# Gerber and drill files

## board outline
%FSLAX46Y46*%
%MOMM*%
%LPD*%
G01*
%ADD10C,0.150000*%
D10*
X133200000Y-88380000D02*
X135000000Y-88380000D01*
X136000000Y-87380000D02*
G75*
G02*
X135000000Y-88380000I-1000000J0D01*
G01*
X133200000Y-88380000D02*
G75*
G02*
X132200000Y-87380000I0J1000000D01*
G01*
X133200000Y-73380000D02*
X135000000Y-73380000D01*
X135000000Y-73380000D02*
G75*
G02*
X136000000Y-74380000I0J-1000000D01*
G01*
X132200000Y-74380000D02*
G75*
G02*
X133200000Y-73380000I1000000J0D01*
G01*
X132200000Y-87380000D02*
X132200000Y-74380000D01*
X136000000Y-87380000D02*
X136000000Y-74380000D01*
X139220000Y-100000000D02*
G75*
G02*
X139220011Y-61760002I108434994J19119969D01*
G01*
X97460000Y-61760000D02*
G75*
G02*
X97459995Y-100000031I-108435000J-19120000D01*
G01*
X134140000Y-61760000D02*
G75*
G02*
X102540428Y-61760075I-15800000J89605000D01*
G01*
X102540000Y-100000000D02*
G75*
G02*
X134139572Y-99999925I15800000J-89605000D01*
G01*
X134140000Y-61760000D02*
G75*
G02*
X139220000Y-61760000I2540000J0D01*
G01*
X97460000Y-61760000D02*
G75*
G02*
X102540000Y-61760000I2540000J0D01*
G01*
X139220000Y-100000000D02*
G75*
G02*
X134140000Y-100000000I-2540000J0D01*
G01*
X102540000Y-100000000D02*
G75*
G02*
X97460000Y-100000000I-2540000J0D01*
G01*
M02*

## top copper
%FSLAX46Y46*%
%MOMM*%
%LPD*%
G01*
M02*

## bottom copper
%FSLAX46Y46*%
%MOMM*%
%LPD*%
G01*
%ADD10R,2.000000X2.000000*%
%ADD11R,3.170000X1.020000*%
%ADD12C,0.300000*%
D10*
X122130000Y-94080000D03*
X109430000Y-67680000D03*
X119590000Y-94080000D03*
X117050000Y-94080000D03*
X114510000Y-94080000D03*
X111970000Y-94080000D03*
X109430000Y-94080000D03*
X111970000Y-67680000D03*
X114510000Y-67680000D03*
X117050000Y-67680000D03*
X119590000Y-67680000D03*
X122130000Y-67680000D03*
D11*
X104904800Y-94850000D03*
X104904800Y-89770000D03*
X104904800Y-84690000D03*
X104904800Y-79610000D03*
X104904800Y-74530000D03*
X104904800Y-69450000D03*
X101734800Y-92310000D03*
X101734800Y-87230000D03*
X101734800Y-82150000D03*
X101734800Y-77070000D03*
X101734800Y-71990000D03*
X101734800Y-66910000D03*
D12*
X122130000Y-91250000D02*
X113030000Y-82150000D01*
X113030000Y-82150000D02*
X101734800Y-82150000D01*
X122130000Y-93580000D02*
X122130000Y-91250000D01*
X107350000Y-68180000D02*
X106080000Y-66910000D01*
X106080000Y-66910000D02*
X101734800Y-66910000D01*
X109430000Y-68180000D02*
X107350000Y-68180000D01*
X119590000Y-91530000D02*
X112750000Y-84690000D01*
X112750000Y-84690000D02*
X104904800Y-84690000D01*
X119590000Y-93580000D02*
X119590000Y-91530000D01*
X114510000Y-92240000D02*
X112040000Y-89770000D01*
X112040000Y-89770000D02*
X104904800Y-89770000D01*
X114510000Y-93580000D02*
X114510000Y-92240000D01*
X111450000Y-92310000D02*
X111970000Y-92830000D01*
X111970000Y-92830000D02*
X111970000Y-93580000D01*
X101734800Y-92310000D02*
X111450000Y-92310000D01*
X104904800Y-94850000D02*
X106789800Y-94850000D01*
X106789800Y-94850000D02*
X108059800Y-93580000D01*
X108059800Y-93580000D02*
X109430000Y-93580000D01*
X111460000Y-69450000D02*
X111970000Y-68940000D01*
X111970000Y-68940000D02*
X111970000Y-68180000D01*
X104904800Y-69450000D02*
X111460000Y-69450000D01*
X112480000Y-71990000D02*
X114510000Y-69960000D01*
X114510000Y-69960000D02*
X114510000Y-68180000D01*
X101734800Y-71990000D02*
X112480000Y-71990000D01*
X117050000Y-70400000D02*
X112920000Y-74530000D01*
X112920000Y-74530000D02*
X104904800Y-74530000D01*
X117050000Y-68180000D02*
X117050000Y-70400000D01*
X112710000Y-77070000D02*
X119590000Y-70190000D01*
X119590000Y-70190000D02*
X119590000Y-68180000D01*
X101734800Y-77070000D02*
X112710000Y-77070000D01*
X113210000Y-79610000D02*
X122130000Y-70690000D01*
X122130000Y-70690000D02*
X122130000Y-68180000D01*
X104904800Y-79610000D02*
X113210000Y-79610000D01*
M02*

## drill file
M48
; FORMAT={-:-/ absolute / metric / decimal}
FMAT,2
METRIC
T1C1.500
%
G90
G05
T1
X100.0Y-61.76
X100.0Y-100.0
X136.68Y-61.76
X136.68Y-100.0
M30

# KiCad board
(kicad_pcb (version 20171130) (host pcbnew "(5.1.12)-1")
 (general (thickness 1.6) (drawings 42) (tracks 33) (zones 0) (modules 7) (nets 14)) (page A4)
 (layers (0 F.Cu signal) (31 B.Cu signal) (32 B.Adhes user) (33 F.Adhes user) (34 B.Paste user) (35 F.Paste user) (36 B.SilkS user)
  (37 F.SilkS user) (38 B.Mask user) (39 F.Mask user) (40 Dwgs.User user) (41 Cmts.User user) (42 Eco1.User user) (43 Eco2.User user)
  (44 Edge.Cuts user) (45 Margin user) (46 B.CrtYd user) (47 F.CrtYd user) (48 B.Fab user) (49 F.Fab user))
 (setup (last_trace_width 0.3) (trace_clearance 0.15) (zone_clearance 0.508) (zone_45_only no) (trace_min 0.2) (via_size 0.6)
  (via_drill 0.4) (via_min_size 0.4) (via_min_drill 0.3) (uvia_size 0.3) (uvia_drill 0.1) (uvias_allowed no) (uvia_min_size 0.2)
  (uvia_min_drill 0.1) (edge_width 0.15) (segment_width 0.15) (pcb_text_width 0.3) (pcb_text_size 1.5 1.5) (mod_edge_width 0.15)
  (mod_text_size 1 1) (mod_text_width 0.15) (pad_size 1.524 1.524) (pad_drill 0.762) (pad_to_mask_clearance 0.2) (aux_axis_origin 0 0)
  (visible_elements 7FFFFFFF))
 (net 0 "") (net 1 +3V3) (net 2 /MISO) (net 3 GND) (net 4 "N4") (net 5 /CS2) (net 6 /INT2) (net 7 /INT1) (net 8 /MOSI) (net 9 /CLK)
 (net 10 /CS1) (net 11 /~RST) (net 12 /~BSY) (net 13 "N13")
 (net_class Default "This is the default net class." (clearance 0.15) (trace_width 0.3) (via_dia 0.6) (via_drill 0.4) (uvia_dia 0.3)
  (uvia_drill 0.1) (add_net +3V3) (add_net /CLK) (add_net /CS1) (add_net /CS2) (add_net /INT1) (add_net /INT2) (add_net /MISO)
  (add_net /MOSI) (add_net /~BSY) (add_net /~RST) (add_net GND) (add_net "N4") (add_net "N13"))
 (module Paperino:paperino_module (layer B.Cu) (at 118.73 80.88 90)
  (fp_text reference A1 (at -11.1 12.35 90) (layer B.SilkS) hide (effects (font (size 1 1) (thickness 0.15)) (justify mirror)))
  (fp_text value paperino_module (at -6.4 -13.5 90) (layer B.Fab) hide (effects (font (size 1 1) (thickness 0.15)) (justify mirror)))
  (pad 1 smd rect (at -12.7 3.4 90) (size 2 2) (drill (offset -0.5 0)) (layers B.Cu B.Paste B.Mask) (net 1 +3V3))
  (pad 7 smd rect (at 12.7 -9.3 90) (size 2 2) (drill (offset 0.5 0)) (layers B.Cu B.Paste B.Mask) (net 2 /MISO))
  (pad 2 smd rect (at -12.7 0.86 90) (size 2 2) (drill (offset -0.5 0)) (layers B.Cu B.Paste B.Mask) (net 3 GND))
  (pad 3 smd rect (at -12.7 -1.68 90) (size 2 2) (drill (offset -0.5 0)) (layers B.Cu B.Paste B.Mask) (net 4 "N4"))
  (pad 4 smd rect (at -12.7 -4.22 90) (size 2 2) (drill (offset -0.5 0)) (layers B.Cu B.Paste B.Mask) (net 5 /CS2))
  (pad 5 smd rect (at -12.7 -6.76 90) (size 2 2) (drill (offset -0.5 0)) (layers B.Cu B.Paste B.Mask) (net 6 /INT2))
  (pad 6 smd rect (at -12.7 -9.3 90) (size 2 2) (drill (offset -0.5 0)) (layers B.Cu B.Paste B.Mask) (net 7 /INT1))
  (pad 8 smd rect (at 12.7 -6.76 90) (size 2 2) (drill (offset 0.5 0)) (layers B.Cu B.Paste B.Mask) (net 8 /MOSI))
  (pad 9 smd rect (at 12.7 -4.22 90) (size 2 2) (drill (offset 0.5 0)) (layers B.Cu B.Paste B.Mask) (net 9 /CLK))
  (pad 10 smd rect (at 12.7 -1.68 90) (size 2 2) (drill (offset 0.5 0)) (layers B.Cu B.Paste B.Mask) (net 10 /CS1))
  (pad 11 smd rect (at 12.7 0.86 90) (size 2 2) (drill (offset 0.5 0)) (layers B.Cu B.Paste B.Mask) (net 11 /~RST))
  (pad 12 smd rect (at 12.7 3.4 90) (size 2 2) (drill (offset 0.5 0)) (layers B.Cu B.Paste B.Mask) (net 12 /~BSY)))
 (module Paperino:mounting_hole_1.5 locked (layer F.Cu) (at 100 100)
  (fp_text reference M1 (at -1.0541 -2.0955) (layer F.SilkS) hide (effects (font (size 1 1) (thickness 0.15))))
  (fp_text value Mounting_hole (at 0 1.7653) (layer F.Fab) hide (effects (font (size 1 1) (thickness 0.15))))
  (pad "" np_thru_hole circle (at 0 0) (size 1.5 1.5) (drill 1.5) (layers *.Cu *.Mask)))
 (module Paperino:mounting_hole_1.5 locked (layer F.Cu) (at 136.68 100)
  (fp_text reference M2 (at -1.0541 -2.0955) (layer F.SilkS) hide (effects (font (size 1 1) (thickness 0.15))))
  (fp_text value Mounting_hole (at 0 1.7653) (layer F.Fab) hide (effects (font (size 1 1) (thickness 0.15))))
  (pad "" np_thru_hole circle (at 0 0) (size 1.5 1.5) (drill 1.5) (layers *.Cu *.Mask)))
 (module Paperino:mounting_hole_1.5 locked (layer F.Cu) (at 100 61.76)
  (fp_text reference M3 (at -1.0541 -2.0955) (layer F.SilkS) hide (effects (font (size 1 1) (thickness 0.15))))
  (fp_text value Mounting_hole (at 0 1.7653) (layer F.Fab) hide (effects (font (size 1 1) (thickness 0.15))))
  (pad "" np_thru_hole circle (at 0 0) (size 1.5 1.5) (drill 1.5) (layers *.Cu *.Mask)))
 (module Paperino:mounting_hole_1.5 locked (layer F.Cu) (at 136.68 61.76)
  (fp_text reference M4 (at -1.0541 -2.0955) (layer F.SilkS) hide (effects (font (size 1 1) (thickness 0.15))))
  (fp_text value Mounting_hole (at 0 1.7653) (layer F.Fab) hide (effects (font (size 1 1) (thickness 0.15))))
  (pad "" np_thru_hole circle (at 0 0) (size 1.5 1.5) (drill 1.5) (layers *.Cu *.Mask)))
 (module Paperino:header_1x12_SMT (layer B.Cu) (at 103.32 80.88 90)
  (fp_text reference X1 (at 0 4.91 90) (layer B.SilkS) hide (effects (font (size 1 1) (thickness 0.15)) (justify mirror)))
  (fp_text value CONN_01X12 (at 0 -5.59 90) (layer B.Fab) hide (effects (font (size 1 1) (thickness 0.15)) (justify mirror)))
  (pad 1 smd rect (at -13.97 1.5848 90) (size 1.02 3.17) (layers B.Cu B.Paste B.Mask) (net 7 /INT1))
  (pad 3 smd rect (at -8.89 1.5848 90) (size 1.02 3.17) (layers B.Cu B.Paste B.Mask) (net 5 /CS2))
  (pad 5 smd rect (at -3.81 1.5848 90) (size 1.02 3.17) (layers B.Cu B.Paste B.Mask) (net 3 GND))
  (pad 7 smd rect (at 1.27 1.5848 90) (size 1.02 3.17) (layers B.Cu B.Paste B.Mask) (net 12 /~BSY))
  (pad 9 smd rect (at 6.35 1.5848 90) (size 1.02 3.17) (layers B.Cu B.Paste B.Mask) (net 10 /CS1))
  (pad 11 smd rect (at 11.43 1.5848 90) (size 1.02 3.17) (layers B.Cu B.Paste B.Mask) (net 8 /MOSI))
  (pad 2 smd rect (at -11.43 -1.5852 90) (size 1.02 3.17) (layers B.Cu B.Paste B.Mask) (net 6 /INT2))
  (pad 4 smd rect (at -6.35 -1.5852 90) (size 1.02 3.17) (layers B.Cu B.Paste B.Mask) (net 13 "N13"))
  (pad 6 smd rect (at -1.27 -1.5852 90) (size 1.02 3.17) (layers B.Cu B.Paste B.Mask) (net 1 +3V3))
  (pad 8 smd rect (at 3.81 -1.5852 90) (size 1.02 3.17) (layers B.Cu B.Paste B.Mask) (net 11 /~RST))
  (pad 10 smd rect (at 8.89 -1.5852 90) (size 1.02 3.17) (layers B.Cu B.Paste B.Mask) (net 9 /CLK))
  (pad 12 smd rect (at 13.97 -1.5852 90) (size 1.02 3.17) (layers B.Cu B.Paste B.Mask) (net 2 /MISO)))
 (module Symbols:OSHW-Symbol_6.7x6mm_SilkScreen (layer F.Cu) (at 133.66 67.9 90)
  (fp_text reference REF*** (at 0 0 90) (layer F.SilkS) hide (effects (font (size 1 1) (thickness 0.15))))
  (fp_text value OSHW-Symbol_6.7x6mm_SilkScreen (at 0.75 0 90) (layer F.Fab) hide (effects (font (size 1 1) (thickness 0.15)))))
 (gr_line (start 133.2 88.38) (end 135 88.38) (layer Edge.Cuts) (width 0.15))
 (gr_arc (start 135 87.38) (end 136 87.38) (angle 90) (layer Edge.Cuts) (width 0.15))
 (gr_arc (start 133.2 87.38) (end 133.2 88.38) (angle 90) (layer Edge.Cuts) (width 0.15))
 (gr_line (start 133.2 73.38) (end 135 73.38) (layer Edge.Cuts) (width 0.15))
 (gr_arc (start 135 74.38) (end 135 73.38) (angle 90) (layer Edge.Cuts) (width 0.15))
 (gr_arc (start 133.2 74.38) (end 132.2 74.38) (angle 90) (layer Edge.Cuts) (width 0.15))
 (gr_line (start 132.2 87.38) (end 132.2 74.38) (layer Edge.Cuts) (width 0.15))
 (gr_line (start 136 87.38) (end 136 74.38) (layer Edge.Cuts) (width 0.15))
 (gr_arc (start 247.654994 80.880031) (end 139.22 100) (angle 19.9999845) (layer Edge.Cuts) (width 0.15))
 (gr_arc (start -10.975 80.88) (end 97.46 61.76) (angle 20) (layer Edge.Cuts) (width 0.15))
 (gr_arc (start 118.34 -27.845) (end 134.14 61.76) (angle 20) (layer Edge.Cuts) (width 0.15))
 (gr_arc (start 118.34 189.605) (end 102.54 100) (angle 20) (layer Edge.Cuts) (width 0.15))
 (gr_arc (start 136.68 61.76) (end 134.14 61.76) (angle 180) (layer Edge.Cuts) (width 0.15))
 (gr_arc (start 100 61.76) (end 97.46 61.76) (angle 180) (layer Edge.Cuts) (width 0.15))
 (gr_arc (start 136.68 100) (end 139.22 100) (angle 180) (layer Edge.Cuts) (width 0.15))
 (gr_arc (start 100 100) (end 102.54 100) (angle 180) (layer Edge.Cuts) (width 0.15))
 (segment (start 122.13 91.25) (end 113.03 82.15) (width 0.3) (layer B.Cu) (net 1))
 (segment (start 113.03 82.15) (end 101.7348 82.15) (width 0.3) (layer B.Cu) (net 1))
 (segment (start 122.13 93.58) (end 122.13 91.25) (width 0.3) (layer B.Cu) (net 1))
 (segment (start 107.35 68.18) (end 106.08 66.91) (width 0.3) (layer B.Cu) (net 2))
 (segment (start 106.08 66.91) (end 101.7348 66.91) (width 0.3) (layer B.Cu) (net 2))
 (segment (start 109.43 68.18) (end 107.35 68.18) (width 0.3) (layer B.Cu) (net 2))
 (segment (start 119.59 91.53) (end 112.75 84.69) (width 0.3) (layer B.Cu) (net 3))
 (segment (start 112.75 84.69) (end 104.9048 84.69) (width 0.3) (layer B.Cu) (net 3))
 (segment (start 119.59 93.58) (end 119.59 91.53) (width 0.3) (layer B.Cu) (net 3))
 (segment (start 114.51 92.24) (end 112.04 89.77) (width 0.3) (layer B.Cu) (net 5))
 (segment (start 112.04 89.77) (end 104.9048 89.77) (width 0.3) (layer B.Cu) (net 5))
 (segment (start 114.51 93.58) (end 114.51 92.24) (width 0.3) (layer B.Cu) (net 5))
 (segment (start 111.45 92.31) (end 111.97 92.83) (width 0.3) (layer B.Cu) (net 6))
 (segment (start 111.97 92.83) (end 111.97 93.58) (width 0.3) (layer B.Cu) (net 6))
 (segment (start 101.7348 92.31) (end 111.45 92.31) (width 0.3) (layer B.Cu) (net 6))
 (segment (start 104.9048 94.85) (end 106.7898 94.85) (width 0.3) (layer B.Cu) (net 7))
 (segment (start 106.7898 94.85) (end 108.0598 93.58) (width 0.3) (layer B.Cu) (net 7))
 (segment (start 108.0598 93.58) (end 109.43 93.58) (width 0.3) (layer B.Cu) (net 7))
 (segment (start 111.46 69.45) (end 111.97 68.94) (width 0.3) (layer B.Cu) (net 8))
 (segment (start 111.97 68.94) (end 111.97 68.18) (width 0.3) (layer B.Cu) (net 8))
 (segment (start 104.9048 69.45) (end 111.46 69.45) (width 0.3) (layer B.Cu) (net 8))
 (segment (start 112.48 71.99) (end 114.51 69.96) (width 0.3) (layer B.Cu) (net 9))
 (segment (start 114.51 69.96) (end 114.51 68.18) (width 0.3) (layer B.Cu) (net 9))
 (segment (start 101.7348 71.99) (end 112.48 71.99) (width 0.3) (layer B.Cu) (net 9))
 (segment (start 117.05 70.4) (end 112.92 74.53) (width 0.3) (layer B.Cu) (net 10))
 (segment (start 112.92 74.53) (end 104.9048 74.53) (width 0.3) (layer B.Cu) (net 10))
 (segment (start 117.05 68.18) (end 117.05 70.4) (width 0.3) (layer B.Cu) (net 10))
 (segment (start 112.71 77.07) (end 119.59 70.19) (width 0.3) (layer B.Cu) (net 11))
 (segment (start 119.59 70.19) (end 119.59 68.18) (width 0.3) (layer B.Cu) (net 11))
 (segment (start 101.7348 77.07) (end 112.71 77.07) (width 0.3) (layer B.Cu) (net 11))
 (segment (start 113.21 79.61) (end 122.13 70.69) (width 0.3) (layer B.Cu) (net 12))
 (segment (start 122.13 70.69) (end 122.13 68.18) (width 0.3) (layer B.Cu) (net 12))
 (segment (start 104.9048 79.61) (end 113.21 79.61) (width 0.3) (layer B.Cu) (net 12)))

